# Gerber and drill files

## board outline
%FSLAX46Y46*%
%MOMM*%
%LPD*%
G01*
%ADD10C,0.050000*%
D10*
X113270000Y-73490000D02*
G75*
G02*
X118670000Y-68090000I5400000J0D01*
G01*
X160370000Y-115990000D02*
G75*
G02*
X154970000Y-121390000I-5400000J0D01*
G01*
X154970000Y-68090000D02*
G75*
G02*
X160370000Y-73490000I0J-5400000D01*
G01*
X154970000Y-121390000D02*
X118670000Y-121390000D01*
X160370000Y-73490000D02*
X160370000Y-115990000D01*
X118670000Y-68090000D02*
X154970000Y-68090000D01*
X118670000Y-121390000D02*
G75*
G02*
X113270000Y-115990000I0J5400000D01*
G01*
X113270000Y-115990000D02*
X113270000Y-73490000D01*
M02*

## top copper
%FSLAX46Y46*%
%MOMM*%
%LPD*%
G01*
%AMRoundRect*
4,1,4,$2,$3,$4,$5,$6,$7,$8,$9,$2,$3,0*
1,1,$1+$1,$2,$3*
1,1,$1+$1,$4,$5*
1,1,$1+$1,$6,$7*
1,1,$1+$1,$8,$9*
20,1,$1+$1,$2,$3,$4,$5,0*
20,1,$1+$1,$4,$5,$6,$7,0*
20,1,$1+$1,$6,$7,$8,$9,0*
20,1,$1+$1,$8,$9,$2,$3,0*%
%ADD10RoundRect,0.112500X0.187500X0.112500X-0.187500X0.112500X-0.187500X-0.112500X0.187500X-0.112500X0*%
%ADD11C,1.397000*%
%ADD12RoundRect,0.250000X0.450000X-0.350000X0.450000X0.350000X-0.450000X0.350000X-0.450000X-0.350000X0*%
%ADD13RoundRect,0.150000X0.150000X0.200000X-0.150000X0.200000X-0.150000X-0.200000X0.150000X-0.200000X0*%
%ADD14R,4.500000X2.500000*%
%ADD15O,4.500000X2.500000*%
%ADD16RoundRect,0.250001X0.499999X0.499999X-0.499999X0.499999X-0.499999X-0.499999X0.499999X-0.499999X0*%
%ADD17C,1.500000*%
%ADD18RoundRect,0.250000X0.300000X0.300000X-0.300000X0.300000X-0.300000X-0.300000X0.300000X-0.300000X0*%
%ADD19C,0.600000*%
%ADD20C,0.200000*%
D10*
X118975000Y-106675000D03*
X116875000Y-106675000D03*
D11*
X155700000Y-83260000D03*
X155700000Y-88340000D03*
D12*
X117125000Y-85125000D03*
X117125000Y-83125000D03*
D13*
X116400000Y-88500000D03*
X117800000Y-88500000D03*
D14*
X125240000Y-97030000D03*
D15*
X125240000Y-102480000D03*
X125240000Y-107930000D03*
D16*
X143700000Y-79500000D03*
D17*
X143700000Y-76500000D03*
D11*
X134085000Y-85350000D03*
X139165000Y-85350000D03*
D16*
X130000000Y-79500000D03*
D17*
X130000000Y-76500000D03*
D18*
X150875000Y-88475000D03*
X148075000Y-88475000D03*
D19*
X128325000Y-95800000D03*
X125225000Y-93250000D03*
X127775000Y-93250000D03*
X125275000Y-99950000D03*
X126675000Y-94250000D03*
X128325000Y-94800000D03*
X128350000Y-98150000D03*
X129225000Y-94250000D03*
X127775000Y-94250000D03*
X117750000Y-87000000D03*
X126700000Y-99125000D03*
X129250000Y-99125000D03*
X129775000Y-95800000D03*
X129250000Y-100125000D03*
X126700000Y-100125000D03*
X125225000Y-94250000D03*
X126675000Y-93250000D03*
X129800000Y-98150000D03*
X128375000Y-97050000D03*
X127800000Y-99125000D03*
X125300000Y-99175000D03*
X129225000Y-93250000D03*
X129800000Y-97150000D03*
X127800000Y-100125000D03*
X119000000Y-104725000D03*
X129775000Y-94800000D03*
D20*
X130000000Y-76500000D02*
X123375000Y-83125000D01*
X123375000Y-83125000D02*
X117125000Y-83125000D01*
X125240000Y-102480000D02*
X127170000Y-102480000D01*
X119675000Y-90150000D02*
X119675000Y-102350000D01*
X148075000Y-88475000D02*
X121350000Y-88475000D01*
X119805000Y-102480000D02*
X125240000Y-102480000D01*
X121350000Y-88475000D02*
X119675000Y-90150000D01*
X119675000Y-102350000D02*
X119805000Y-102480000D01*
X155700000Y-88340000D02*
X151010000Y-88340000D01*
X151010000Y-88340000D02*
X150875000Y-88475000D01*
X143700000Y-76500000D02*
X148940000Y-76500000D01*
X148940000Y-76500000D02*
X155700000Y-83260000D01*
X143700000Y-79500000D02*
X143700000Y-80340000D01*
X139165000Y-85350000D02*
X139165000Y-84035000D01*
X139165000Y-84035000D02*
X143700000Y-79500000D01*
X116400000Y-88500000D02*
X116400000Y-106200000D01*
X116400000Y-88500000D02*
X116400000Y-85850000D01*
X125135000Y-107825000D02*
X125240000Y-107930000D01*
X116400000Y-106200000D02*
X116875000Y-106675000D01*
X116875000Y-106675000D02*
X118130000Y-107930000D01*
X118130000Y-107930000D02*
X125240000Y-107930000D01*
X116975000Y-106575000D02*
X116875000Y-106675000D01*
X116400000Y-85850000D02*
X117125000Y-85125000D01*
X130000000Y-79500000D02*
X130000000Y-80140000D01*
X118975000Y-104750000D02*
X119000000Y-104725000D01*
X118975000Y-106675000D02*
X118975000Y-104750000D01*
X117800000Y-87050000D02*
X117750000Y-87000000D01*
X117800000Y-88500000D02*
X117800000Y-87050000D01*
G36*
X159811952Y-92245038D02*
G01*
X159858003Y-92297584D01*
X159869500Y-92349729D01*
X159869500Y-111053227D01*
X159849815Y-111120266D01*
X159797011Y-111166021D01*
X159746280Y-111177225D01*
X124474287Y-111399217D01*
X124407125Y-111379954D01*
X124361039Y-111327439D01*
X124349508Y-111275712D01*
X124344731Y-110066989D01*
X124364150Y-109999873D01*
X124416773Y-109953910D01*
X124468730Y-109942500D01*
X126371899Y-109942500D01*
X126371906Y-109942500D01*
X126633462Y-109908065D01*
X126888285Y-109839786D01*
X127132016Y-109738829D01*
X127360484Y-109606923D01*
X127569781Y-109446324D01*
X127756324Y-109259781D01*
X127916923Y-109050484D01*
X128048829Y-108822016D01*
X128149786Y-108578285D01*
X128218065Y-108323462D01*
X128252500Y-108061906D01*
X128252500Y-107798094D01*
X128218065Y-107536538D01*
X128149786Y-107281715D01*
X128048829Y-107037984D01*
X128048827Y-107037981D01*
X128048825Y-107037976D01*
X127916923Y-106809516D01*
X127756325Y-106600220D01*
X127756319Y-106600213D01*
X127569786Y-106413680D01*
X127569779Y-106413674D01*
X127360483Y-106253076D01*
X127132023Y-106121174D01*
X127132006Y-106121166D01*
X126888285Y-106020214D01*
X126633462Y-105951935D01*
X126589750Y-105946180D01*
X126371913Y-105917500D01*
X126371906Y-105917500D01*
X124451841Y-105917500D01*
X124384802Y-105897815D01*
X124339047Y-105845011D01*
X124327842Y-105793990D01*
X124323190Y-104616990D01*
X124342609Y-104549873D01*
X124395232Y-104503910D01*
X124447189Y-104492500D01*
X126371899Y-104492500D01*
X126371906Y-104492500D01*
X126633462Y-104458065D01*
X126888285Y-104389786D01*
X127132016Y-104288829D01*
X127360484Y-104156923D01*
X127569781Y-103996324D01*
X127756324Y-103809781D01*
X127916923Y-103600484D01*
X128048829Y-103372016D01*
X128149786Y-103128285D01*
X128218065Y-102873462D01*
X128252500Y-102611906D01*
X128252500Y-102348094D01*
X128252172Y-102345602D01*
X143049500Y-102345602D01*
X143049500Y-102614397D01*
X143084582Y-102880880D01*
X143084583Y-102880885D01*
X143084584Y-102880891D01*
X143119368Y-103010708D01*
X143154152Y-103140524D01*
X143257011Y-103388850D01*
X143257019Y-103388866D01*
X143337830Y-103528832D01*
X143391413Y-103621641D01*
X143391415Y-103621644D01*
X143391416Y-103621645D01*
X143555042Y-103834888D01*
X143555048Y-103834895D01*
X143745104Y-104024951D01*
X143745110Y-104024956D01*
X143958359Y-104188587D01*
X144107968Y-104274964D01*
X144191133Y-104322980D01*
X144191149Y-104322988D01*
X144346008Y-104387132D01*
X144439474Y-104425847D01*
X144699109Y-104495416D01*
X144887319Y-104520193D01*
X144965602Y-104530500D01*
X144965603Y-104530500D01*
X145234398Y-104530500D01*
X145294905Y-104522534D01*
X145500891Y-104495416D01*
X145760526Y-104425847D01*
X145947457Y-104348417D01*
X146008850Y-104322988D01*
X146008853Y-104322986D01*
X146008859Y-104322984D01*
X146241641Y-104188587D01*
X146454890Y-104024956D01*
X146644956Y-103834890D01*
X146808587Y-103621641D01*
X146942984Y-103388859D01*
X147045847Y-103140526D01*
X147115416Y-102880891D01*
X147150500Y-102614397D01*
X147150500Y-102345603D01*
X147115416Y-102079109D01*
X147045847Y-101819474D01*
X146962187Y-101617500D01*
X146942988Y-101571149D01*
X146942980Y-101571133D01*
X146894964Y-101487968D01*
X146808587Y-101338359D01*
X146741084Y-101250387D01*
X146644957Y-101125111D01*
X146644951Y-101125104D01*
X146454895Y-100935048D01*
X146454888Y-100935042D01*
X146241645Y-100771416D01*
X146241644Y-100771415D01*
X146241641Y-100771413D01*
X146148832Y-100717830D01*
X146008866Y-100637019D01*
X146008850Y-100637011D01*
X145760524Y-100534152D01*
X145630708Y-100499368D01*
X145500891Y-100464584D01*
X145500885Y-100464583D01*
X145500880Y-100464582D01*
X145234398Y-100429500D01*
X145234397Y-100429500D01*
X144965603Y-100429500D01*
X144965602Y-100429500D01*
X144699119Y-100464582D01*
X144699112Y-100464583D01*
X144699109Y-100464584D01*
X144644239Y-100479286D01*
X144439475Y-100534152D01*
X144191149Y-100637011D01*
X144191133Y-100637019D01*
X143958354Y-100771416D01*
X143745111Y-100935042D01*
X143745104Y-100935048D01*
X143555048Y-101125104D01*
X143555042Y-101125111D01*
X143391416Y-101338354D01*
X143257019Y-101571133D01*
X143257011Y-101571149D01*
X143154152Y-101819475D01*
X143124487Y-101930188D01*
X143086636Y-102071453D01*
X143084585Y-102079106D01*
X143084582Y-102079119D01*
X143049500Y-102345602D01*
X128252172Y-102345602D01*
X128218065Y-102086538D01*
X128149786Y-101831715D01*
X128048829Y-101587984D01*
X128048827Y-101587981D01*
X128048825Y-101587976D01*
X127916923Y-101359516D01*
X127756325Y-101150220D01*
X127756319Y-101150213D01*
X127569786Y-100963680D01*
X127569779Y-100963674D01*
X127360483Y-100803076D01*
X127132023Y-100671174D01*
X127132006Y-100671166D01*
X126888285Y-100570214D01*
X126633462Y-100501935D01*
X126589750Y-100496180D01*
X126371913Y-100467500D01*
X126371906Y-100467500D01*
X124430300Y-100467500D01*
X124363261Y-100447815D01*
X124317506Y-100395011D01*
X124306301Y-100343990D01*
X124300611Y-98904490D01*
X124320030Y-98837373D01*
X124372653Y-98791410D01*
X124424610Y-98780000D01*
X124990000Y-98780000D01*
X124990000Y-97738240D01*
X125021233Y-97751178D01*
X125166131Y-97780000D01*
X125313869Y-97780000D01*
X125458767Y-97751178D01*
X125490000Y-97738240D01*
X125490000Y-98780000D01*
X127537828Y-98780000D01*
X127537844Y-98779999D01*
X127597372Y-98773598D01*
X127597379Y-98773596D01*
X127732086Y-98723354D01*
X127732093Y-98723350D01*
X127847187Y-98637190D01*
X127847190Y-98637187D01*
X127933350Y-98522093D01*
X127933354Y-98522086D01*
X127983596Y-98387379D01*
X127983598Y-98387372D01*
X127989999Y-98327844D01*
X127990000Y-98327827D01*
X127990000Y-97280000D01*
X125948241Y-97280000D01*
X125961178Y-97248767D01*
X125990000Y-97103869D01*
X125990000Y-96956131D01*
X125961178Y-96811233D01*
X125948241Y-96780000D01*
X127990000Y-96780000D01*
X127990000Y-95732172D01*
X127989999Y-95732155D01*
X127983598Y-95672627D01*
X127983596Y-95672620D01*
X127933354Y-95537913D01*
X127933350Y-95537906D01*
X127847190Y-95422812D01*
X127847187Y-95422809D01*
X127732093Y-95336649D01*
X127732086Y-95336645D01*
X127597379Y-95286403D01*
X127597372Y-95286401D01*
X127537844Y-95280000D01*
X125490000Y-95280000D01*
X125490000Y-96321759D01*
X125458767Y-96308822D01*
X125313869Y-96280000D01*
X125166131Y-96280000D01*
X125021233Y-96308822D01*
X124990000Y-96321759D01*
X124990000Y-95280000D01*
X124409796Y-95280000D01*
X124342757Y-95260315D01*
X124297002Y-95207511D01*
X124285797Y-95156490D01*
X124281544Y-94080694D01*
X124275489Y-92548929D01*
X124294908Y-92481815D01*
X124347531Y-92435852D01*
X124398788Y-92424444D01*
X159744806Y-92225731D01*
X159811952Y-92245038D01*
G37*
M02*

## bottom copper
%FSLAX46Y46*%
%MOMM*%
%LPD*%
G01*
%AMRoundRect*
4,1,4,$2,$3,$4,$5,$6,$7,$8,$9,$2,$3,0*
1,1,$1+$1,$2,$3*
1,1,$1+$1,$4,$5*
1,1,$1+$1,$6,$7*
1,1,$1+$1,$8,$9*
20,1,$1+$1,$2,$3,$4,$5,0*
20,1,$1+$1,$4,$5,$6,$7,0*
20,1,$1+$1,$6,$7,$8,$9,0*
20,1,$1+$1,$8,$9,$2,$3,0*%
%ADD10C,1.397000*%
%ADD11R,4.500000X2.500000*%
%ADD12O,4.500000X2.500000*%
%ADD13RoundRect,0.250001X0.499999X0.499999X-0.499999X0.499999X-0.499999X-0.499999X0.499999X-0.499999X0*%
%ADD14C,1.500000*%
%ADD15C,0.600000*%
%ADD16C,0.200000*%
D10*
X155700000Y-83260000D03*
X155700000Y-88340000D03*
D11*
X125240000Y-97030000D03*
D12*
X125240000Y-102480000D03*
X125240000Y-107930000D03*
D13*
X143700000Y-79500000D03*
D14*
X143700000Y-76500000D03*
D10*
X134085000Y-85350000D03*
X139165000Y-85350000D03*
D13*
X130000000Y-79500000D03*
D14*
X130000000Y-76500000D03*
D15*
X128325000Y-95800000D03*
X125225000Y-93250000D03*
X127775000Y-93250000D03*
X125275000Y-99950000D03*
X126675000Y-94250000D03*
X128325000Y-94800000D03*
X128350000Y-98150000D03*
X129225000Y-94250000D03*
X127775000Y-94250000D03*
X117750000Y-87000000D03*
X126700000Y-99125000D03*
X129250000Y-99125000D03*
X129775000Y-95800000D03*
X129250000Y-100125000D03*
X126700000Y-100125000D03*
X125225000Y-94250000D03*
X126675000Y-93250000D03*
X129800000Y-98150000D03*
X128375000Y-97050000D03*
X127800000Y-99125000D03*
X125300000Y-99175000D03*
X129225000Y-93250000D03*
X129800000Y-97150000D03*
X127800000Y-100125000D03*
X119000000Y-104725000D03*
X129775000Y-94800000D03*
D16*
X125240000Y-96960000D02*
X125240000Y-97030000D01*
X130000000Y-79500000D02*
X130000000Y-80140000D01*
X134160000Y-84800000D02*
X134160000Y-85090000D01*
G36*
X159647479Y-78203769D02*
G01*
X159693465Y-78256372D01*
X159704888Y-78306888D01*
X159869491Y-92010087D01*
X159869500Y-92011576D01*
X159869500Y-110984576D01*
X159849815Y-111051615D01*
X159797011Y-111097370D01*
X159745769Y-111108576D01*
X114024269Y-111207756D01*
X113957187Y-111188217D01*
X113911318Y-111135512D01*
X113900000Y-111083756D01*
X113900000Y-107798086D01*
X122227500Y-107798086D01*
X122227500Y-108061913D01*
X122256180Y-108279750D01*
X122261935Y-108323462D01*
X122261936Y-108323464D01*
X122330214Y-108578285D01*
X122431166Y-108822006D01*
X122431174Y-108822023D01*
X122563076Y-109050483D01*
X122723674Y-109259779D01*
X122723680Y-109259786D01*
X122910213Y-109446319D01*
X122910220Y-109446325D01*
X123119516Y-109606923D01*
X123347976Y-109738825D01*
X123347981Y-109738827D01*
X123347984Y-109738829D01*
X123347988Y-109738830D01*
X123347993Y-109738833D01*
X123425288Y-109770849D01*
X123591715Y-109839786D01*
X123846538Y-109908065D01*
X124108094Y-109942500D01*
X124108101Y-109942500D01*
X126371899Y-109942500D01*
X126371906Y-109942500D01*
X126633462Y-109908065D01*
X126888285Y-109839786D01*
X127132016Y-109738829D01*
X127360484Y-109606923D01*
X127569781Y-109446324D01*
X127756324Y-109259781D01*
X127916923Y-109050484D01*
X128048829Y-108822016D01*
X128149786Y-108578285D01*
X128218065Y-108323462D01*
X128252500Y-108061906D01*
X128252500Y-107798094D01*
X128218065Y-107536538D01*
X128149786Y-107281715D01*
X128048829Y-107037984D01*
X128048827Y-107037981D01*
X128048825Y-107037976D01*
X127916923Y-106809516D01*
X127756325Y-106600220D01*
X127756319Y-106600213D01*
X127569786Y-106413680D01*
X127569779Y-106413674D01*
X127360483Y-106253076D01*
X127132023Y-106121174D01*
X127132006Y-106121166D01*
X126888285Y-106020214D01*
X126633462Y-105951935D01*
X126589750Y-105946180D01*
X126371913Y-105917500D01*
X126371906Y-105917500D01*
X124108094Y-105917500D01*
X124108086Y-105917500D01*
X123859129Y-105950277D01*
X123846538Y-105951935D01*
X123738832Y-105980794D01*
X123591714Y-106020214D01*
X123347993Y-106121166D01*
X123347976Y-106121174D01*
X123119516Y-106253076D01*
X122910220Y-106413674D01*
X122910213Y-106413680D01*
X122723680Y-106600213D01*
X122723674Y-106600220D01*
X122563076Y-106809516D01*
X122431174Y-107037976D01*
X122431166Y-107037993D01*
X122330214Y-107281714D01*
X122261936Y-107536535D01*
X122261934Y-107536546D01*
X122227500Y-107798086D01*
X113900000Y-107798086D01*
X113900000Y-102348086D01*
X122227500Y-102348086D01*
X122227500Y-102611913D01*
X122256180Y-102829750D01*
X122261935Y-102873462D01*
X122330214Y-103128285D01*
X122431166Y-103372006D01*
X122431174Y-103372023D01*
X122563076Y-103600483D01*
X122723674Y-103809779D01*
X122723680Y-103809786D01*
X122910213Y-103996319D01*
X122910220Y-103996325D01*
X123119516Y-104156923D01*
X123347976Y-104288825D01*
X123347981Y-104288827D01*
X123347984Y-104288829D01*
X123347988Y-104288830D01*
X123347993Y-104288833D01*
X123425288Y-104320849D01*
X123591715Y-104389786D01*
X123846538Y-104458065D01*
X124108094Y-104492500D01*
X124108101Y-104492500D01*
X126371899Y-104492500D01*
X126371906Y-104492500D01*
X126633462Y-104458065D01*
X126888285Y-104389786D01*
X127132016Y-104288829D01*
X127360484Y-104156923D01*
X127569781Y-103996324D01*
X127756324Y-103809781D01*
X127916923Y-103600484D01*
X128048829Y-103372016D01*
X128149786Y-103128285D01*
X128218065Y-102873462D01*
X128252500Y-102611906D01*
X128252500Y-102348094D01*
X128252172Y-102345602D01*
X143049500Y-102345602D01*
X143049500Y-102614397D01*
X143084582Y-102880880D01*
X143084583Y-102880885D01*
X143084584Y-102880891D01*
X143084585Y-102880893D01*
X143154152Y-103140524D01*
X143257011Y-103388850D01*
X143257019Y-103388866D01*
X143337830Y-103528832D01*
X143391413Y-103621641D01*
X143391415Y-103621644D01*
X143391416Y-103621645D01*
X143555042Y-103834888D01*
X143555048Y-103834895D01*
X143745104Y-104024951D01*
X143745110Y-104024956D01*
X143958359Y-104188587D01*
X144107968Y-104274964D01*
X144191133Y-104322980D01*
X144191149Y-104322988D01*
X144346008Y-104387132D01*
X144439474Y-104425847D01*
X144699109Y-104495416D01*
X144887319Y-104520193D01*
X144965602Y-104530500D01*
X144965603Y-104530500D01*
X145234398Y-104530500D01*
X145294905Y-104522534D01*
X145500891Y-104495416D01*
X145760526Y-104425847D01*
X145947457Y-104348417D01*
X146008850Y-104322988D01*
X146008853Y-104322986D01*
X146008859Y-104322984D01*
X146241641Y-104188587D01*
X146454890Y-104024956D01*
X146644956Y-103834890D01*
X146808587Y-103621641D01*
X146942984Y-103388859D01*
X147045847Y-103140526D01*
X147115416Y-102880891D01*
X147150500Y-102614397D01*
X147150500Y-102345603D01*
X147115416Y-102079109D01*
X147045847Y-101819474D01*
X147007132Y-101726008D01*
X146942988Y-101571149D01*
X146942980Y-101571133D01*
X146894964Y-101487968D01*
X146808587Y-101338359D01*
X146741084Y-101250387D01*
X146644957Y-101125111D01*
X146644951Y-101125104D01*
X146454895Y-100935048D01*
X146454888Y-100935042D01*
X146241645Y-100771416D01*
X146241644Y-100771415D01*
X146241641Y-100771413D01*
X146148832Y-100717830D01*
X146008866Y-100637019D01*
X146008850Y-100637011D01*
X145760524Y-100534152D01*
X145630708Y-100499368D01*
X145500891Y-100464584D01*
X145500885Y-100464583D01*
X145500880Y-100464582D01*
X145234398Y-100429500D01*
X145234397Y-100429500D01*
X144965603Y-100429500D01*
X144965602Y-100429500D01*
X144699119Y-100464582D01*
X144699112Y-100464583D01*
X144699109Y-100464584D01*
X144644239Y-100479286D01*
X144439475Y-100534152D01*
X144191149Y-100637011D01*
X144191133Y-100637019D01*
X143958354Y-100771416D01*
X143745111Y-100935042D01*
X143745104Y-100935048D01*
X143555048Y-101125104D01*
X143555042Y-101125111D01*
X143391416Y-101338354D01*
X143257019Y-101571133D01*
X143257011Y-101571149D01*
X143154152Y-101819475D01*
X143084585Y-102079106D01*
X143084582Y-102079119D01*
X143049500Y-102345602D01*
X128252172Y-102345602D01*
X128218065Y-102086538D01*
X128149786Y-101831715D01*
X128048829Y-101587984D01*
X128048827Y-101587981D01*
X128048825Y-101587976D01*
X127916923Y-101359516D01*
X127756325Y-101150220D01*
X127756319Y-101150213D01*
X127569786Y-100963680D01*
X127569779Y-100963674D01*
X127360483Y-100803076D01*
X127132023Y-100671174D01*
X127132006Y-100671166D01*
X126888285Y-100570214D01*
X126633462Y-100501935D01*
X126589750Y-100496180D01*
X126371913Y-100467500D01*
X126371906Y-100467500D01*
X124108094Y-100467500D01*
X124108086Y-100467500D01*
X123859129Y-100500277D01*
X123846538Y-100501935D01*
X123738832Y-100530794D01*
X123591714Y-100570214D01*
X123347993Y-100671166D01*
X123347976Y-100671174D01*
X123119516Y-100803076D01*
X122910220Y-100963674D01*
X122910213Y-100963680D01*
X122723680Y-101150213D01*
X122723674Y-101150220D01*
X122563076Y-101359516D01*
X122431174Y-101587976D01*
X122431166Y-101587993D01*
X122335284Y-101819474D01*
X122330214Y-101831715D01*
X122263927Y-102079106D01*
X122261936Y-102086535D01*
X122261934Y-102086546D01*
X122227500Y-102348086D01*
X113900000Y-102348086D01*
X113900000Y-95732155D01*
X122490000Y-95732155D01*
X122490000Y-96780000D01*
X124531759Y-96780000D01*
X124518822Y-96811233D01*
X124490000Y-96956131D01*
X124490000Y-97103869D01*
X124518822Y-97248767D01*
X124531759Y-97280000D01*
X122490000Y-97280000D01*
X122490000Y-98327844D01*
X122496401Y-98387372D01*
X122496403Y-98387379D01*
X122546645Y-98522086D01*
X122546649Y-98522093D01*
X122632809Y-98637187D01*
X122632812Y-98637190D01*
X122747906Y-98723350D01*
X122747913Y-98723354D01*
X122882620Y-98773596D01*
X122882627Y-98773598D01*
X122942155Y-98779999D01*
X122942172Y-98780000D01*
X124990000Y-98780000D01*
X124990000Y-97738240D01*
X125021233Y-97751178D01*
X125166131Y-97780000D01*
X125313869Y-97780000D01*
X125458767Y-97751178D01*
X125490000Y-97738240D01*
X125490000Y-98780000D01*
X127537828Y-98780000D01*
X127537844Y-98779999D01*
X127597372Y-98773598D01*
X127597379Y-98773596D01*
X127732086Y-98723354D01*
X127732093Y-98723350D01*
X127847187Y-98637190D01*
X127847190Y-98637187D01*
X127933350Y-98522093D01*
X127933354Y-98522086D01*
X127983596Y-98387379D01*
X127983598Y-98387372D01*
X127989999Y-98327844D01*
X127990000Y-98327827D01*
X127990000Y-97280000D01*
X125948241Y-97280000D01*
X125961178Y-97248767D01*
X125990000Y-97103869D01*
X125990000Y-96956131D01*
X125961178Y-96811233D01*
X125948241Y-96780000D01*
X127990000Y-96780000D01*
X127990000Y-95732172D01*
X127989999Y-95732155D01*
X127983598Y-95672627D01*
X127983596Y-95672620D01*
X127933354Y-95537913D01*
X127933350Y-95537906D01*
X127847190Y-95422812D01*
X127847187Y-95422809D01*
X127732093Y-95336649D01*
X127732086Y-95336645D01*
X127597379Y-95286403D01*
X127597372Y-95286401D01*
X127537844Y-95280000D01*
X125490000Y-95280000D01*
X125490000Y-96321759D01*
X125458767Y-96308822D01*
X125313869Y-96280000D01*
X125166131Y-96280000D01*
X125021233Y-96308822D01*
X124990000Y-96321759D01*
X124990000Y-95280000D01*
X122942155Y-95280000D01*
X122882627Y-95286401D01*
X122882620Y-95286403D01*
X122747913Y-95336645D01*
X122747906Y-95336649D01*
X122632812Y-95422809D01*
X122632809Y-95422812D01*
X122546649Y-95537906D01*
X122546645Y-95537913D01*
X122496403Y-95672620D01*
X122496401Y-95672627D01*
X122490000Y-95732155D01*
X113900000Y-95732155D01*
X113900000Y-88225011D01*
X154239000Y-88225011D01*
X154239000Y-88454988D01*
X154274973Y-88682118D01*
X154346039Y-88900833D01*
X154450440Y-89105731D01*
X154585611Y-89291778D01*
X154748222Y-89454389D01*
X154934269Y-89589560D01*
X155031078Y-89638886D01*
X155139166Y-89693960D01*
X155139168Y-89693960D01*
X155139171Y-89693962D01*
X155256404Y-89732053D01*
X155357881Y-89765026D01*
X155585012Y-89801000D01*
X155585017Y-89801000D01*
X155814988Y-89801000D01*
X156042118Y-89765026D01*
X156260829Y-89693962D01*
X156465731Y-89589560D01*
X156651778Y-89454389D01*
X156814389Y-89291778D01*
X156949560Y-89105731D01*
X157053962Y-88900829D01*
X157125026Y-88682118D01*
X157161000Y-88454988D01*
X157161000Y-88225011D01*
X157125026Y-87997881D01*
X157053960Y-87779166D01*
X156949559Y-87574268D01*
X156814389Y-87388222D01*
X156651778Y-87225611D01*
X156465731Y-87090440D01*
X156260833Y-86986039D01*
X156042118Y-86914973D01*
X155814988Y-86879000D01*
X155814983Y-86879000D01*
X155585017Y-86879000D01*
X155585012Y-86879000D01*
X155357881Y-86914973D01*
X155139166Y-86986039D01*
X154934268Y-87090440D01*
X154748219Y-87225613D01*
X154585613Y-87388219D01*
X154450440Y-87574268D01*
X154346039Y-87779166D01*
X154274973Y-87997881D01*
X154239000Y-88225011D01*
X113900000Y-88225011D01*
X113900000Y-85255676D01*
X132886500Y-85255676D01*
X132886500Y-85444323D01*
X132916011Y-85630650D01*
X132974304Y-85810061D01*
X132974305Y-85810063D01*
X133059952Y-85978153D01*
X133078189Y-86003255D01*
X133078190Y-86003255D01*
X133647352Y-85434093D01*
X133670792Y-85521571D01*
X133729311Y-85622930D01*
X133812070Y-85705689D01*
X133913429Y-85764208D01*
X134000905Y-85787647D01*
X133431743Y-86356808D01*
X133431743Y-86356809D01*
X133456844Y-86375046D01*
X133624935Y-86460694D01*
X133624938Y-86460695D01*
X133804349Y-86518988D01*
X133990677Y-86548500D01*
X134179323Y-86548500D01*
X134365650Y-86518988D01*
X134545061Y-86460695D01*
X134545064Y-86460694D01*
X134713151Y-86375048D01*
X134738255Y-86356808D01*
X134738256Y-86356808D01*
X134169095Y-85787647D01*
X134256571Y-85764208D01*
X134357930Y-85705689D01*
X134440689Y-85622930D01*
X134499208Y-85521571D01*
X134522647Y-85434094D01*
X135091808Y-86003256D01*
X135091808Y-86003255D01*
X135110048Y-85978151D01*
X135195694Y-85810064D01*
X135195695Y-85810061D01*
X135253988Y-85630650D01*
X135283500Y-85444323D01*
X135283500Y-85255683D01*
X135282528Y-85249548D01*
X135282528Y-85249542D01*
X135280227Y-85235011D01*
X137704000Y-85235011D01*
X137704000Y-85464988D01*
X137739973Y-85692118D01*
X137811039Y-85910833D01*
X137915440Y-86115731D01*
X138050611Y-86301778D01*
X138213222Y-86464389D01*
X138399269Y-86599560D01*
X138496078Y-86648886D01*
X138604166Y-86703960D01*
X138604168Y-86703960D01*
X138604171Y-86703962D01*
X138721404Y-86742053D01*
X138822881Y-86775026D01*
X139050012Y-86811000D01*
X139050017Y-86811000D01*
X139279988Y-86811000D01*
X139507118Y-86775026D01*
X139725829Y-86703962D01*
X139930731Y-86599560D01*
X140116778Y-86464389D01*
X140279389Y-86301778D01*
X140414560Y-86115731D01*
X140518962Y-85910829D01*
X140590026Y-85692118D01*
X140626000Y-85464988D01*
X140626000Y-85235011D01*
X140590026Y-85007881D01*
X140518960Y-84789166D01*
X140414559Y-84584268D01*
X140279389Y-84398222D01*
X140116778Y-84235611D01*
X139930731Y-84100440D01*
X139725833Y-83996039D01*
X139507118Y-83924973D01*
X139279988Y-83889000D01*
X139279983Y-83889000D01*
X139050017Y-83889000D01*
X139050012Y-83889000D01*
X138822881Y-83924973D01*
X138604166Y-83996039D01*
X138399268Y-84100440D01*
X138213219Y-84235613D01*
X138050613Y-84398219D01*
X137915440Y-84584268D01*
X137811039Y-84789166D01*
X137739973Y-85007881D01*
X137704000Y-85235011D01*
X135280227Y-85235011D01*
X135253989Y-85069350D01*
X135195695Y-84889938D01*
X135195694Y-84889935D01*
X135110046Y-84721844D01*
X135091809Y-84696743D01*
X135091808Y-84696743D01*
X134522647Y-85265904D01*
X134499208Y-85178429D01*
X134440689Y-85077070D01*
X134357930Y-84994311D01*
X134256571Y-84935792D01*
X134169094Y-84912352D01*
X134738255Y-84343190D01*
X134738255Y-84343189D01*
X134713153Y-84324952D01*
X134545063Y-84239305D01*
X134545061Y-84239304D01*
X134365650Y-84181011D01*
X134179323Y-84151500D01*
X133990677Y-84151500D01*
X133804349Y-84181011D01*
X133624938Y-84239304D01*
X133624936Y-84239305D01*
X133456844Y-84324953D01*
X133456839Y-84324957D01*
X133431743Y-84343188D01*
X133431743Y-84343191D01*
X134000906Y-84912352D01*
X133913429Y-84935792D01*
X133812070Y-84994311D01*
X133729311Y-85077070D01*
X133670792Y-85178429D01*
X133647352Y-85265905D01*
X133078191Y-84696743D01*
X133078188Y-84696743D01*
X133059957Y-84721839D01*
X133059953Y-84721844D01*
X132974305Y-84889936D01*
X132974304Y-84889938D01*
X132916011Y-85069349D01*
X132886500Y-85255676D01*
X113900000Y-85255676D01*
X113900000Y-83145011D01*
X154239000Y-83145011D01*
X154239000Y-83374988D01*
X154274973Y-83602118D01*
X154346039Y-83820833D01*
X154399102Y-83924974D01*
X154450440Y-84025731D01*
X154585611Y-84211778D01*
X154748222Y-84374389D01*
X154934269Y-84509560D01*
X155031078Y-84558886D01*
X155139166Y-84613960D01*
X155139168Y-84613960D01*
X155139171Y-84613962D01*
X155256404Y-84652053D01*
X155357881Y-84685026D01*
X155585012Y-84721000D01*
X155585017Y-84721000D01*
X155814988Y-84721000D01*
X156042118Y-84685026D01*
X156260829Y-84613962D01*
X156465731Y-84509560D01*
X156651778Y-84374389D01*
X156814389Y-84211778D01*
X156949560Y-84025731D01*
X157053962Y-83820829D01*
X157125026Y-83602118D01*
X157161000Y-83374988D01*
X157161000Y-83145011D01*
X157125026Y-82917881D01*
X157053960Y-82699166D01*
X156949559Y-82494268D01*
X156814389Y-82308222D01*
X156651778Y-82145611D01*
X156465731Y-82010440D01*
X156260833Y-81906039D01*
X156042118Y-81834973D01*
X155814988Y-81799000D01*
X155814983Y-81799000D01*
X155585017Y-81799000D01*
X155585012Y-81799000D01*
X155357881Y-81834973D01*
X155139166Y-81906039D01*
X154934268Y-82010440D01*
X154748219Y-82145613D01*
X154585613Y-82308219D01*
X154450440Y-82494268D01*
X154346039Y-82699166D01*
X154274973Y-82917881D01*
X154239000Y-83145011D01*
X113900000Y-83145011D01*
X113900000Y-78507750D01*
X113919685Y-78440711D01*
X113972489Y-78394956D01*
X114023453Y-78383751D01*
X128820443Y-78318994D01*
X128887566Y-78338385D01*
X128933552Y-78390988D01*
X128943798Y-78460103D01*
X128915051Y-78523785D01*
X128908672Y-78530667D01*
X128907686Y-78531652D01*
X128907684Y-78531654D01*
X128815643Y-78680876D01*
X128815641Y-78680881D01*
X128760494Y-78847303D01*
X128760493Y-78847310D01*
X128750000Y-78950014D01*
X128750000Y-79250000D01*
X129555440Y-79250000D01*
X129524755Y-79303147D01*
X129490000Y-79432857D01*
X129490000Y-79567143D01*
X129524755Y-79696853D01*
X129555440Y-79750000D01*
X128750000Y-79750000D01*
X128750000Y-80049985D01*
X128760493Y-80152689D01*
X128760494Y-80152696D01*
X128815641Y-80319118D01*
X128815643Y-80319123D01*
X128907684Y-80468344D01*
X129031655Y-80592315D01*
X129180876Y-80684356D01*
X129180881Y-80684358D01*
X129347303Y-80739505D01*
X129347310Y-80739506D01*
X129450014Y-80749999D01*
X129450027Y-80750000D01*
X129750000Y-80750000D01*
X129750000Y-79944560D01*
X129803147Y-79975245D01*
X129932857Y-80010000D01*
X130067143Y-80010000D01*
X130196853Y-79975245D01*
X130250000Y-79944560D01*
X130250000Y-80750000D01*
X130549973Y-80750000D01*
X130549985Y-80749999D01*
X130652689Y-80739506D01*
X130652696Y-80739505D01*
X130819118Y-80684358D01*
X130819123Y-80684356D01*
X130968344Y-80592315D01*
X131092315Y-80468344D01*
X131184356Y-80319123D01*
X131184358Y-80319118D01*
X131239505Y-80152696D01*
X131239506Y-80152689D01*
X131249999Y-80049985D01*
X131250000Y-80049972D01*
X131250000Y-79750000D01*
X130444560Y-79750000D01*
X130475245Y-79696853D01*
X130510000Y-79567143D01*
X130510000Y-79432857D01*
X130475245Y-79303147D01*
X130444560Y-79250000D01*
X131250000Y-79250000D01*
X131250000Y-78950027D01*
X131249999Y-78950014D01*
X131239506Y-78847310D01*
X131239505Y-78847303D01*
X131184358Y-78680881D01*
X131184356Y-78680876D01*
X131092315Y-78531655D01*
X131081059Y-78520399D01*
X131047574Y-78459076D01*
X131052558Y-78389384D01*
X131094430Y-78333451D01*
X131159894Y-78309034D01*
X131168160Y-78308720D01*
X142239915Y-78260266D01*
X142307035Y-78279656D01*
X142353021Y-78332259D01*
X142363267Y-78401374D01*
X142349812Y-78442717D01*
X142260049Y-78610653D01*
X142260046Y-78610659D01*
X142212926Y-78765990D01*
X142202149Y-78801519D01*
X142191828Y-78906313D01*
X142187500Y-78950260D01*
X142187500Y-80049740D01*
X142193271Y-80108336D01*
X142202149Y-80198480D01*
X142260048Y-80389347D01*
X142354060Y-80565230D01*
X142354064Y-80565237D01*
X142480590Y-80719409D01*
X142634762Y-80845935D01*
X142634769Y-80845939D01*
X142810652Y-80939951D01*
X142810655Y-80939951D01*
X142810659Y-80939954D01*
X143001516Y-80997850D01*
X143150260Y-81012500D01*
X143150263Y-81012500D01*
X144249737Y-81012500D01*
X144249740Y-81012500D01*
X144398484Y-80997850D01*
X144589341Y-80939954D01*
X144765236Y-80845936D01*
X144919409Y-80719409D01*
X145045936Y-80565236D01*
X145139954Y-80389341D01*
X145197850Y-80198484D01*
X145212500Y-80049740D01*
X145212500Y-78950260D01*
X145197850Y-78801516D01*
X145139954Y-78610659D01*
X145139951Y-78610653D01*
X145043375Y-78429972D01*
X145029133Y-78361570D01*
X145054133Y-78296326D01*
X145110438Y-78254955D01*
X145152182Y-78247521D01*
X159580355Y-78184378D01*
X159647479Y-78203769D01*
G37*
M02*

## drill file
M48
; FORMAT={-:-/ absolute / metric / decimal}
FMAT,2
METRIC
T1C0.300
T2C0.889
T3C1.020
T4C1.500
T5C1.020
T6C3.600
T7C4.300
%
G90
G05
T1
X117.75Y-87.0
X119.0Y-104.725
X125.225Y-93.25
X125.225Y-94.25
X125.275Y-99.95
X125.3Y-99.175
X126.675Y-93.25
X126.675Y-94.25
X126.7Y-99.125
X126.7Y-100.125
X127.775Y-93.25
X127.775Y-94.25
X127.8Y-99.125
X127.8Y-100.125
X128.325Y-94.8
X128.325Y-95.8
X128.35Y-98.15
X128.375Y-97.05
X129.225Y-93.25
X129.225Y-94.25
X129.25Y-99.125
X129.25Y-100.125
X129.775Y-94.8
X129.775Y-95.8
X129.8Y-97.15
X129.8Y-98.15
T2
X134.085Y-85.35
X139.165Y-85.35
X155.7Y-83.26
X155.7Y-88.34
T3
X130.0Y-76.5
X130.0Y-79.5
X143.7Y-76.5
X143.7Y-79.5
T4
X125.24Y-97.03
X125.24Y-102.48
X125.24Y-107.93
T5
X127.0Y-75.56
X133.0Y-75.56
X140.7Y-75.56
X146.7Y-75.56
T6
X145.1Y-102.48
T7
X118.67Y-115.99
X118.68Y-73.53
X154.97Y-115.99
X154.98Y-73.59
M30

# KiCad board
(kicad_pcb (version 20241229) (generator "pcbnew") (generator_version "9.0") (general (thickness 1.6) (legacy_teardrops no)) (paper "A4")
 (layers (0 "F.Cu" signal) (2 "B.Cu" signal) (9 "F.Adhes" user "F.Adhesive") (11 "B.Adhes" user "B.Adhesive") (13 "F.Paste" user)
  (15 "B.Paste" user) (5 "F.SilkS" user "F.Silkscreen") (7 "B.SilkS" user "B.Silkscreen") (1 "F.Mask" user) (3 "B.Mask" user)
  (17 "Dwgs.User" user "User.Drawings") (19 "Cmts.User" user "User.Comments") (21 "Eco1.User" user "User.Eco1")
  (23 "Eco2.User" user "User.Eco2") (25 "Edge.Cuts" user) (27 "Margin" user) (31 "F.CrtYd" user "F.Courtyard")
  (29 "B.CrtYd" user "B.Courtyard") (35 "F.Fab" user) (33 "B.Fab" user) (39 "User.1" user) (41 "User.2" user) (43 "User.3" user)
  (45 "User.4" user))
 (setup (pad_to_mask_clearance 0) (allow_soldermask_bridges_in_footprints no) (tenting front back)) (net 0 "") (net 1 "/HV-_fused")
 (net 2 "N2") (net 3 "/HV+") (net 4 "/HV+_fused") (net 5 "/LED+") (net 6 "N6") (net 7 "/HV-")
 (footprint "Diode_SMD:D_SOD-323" (layer "F.Cu") (at 117.925 106.675 180)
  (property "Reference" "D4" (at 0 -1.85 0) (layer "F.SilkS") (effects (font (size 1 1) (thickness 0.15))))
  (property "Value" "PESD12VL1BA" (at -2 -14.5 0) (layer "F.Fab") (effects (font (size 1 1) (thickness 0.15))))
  (pad "1" smd roundrect (at -1.05 0 180) (size 0.6 0.45) (layers "F.Cu" "F.Mask" "F.Paste") (roundrect_rratio 0.25) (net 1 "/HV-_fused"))
  (pad "2" smd roundrect (at 1.05 0 180) (size 0.6 0.45) (layers "F.Cu" "F.Mask" "F.Paste") (roundrect_rratio 0.25) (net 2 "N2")))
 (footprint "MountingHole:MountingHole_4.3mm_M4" (layer "F.Cu") (at 118.679999 73.53 180)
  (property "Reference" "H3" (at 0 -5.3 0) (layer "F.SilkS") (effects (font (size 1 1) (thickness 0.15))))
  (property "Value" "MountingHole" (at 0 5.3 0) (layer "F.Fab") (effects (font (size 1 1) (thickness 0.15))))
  (pad "" np_thru_hole circle (at 0 0 180) (size 4.3 4.3) (drill 4.3) (layers "*.Cu" "*.Mask")))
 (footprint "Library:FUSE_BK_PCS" (layer "F.Cu") (at 155.7 85.8 -90)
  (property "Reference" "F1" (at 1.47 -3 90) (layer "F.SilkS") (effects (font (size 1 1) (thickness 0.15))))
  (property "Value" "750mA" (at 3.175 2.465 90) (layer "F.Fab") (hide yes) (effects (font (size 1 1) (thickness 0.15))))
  (pad "1" thru_hole circle (at -2.54 0 270) (size 1.397 1.397) (drill 0.889) (layers "*.Cu" "*.Mask") (remove_unused_layers no)
   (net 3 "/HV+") (solder_mask_margin 0.102))
  (pad "2" thru_hole circle (at 2.54 0 270) (size 1.397 1.397) (drill 0.889) (layers "*.Cu" "*.Mask") (remove_unused_layers no)
   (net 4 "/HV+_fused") (solder_mask_margin 0.102)))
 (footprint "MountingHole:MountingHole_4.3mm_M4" (layer "F.Cu") (at 118.669999 115.990001)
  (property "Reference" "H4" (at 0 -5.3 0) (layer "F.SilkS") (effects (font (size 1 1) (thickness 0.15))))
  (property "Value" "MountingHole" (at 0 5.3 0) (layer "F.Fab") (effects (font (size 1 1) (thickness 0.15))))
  (pad "" np_thru_hole circle (at 0 0) (size 4.3 4.3) (drill 4.3) (layers "*.Cu" "*.Mask")))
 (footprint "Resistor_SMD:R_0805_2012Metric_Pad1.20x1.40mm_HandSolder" (layer "F.Cu") (at 117.125 84.125 90)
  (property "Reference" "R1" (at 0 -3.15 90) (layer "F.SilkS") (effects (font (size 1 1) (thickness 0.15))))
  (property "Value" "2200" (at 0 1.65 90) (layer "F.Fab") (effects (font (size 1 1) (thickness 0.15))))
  (pad "1" smd roundrect (at -1 0 90) (size 1.2 1.4) (layers "F.Cu" "F.Mask" "F.Paste") (roundrect_rratio 0.208333) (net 2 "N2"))
  (pad "2" smd roundrect (at 1 0 90) (size 1.2 1.4) (layers "F.Cu" "F.Mask" "F.Paste") (roundrect_rratio 0.208333) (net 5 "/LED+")))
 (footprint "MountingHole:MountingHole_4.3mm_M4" (layer "F.Cu") (at 154.980001 73.59 180)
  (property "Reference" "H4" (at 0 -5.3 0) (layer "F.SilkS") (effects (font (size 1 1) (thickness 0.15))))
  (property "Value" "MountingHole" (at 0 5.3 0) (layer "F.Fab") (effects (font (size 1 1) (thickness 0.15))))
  (pad "" np_thru_hole circle (at 0 0 180) (size 4.3 4.3) (drill 4.3) (layers "*.Cu" "*.Mask")))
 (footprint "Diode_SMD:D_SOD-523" (layer "F.Cu") (at 117.1 88.5)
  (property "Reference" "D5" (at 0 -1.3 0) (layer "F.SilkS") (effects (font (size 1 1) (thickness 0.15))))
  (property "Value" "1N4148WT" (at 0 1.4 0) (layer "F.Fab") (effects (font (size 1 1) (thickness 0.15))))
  (pad "1" smd roundrect (at -0.7 0 180) (size 0.6 0.7) (layers "F.Cu" "F.Mask" "F.Paste") (roundrect_rratio 0.25) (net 2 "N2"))
  (pad "2" smd roundrect (at 0.7 0 180) (size 0.6 0.7) (layers "F.Cu" "F.Mask" "F.Paste") (roundrect_rratio 0.25) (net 1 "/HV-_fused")))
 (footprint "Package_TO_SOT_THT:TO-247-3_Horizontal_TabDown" (layer "F.Cu") (at 125.24 97.03 -90)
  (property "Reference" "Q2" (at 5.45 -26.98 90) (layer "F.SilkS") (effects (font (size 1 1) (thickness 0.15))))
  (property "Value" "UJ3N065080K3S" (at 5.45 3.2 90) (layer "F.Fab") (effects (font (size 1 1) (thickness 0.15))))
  (pad "" np_thru_hole circle (at 5.45 -19.86 270) (size 3.6 3.6) (drill 3.6) (layers "*.Cu" "*.Mask"))
  (pad "1" thru_hole rect (at 0 0 270) (size 2.5 4.5) (drill 1.5) (layers "*.Cu" "*.Mask") (remove_unused_layers no) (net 1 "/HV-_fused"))
  (pad "2" thru_hole oval (at 5.45 0 270) (size 2.5 4.5) (drill 1.5) (layers "*.Cu" "*.Mask") (remove_unused_layers no) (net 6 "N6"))
  (pad "3" thru_hole oval (at 10.9 0 270) (size 2.5 4.5) (drill 1.5) (layers "*.Cu" "*.Mask") (remove_unused_layers no) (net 2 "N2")))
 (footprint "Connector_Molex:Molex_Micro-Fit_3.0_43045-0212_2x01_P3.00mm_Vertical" (layer "F.Cu") (at 143.7 79.5 180)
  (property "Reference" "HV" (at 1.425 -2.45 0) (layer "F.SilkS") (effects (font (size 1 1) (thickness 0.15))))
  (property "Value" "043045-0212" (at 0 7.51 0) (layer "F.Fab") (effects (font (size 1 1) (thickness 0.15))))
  (pad "" np_thru_hole circle (at -3 3.94 180) (size 1.02 1.02) (drill 1.02) (layers "*.Cu" "*.Mask"))
  (pad "" np_thru_hole circle (at 3 3.94 180) (size 1.02 1.02) (drill 1.02) (layers "*.Cu" "*.Mask"))
  (pad "1" thru_hole roundrect (at 0 0 180) (size 1.5 1.5) (drill 1.02) (layers "*.Cu" "*.Mask") (remove_unused_layers no)
   (roundrect_rratio 0.166667) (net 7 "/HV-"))
  (pad "2" thru_hole circle (at 0 3 180) (size 1.5 1.5) (drill 1.02) (layers "*.Cu" "*.Mask") (remove_unused_layers no) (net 3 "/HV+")))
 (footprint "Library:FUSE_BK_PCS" (layer "F.Cu") (at 136.625 85.35)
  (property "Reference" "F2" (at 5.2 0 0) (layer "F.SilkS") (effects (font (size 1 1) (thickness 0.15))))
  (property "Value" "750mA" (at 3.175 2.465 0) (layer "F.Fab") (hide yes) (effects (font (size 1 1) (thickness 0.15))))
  (pad "1" thru_hole circle (at -2.54 0) (size 1.397 1.397) (drill 0.889) (layers "*.Cu" "*.Mask") (remove_unused_layers no)
   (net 1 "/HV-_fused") (solder_mask_margin 0.102))
  (pad "2" thru_hole circle (at 2.54 0) (size 1.397 1.397) (drill 0.889) (layers "*.Cu" "*.Mask") (remove_unused_layers no) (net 7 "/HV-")
   (solder_mask_margin 0.102)))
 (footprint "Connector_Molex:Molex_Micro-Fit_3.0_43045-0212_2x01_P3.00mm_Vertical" (layer "F.Cu") (at 130 79.5 180)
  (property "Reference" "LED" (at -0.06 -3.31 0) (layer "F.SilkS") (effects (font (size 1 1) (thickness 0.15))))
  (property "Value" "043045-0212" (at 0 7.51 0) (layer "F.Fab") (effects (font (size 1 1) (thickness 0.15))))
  (pad "" np_thru_hole circle (at -3 3.94 180) (size 1.02 1.02) (drill 1.02) (layers "*.Cu" "*.Mask"))
  (pad "" np_thru_hole circle (at 3 3.94 180) (size 1.02 1.02) (drill 1.02) (layers "*.Cu" "*.Mask"))
  (pad "1" thru_hole roundrect (at 0 0 180) (size 1.5 1.5) (drill 1.02) (layers "*.Cu" "*.Mask") (remove_unused_layers no)
   (roundrect_rratio 0.166667) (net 1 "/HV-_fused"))
  (pad "2" thru_hole circle (at 0 3 180) (size 1.5 1.5) (drill 1.02) (layers "*.Cu" "*.Mask") (remove_unused_layers no) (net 5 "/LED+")))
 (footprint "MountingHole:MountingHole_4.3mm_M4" (layer "F.Cu") (at 154.970001 115.990001)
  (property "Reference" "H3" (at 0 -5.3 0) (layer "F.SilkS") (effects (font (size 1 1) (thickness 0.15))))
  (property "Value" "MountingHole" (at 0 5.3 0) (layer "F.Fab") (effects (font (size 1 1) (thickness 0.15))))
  (pad "" np_thru_hole circle (at 0 0) (size 4.3 4.3) (drill 4.3) (layers "*.Cu" "*.Mask")))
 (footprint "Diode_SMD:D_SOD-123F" (layer "F.Cu") (at 149.475 88.475 180)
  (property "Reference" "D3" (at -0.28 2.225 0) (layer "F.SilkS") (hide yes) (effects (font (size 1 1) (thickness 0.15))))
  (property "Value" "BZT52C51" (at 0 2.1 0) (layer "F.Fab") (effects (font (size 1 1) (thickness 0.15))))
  (pad "1" smd roundrect (at -1.4 0 180) (size 1.1 1.1) (layers "F.Cu" "F.Mask" "F.Paste") (roundrect_rratio 0.2272727273)
   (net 4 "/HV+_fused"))
  (pad "2" smd roundrect (at 1.4 0 180) (size 1.1 1.1) (layers "F.Cu" "F.Mask" "F.Paste") (roundrect_rratio 0.2272727273) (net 6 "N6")))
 (gr_arc (start 113.27 73.49) (mid 114.851623 69.671623) (end 118.67 68.09) (stroke (width 0.05) (type default)) (layer "Edge.Cuts"))
 (gr_arc (start 160.37 115.99) (mid 158.788377 119.808377) (end 154.97 121.39) (stroke (width 0.05) (type default)) (layer "Edge.Cuts"))
 (gr_arc (start 154.97 68.09) (mid 158.788377 69.671623) (end 160.37 73.49) (stroke (width 0.05) (type default)) (layer "Edge.Cuts"))
 (gr_line (start 154.97 121.39) (end 118.67 121.39) (stroke (width 0.05) (type default)) (layer "Edge.Cuts"))
 (gr_line (start 160.37 73.49) (end 160.37 115.99) (stroke (width 0.05) (type default)) (layer "Edge.Cuts"))
 (gr_line (start 118.67 68.09) (end 154.97 68.09) (stroke (width 0.05) (type default)) (layer "Edge.Cuts"))
 (gr_arc (start 118.67 121.39) (mid 114.851623 119.808377) (end 113.27 115.99) (stroke (width 0.05) (type default)) (layer "Edge.Cuts"))
 (gr_line (start 113.27 115.99) (end 113.27 73.49) (stroke (width 0.05) (type default)) (layer "Edge.Cuts"))
 (segment (start 130 76.5) (end 123.375 83.125) (width 0.2) (layer "F.Cu") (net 5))
 (segment (start 123.375 83.125) (end 117.125 83.125) (width 0.2) (layer "F.Cu") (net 5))
 (segment (start 125.24 102.48) (end 127.17 102.48) (width 0.2) (layer "F.Cu") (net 6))
 (segment (start 119.675 90.15) (end 119.675 102.35) (width 0.2) (layer "F.Cu") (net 6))
 (segment (start 148.075 88.475) (end 121.35 88.475) (width 0.2) (layer "F.Cu") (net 6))
 (segment (start 119.805 102.48) (end 125.24 102.48) (width 0.2) (layer "F.Cu") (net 6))
 (segment (start 121.35 88.475) (end 119.675 90.15) (width 0.2) (layer "F.Cu") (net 6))
 (segment (start 119.675 102.35) (end 119.805 102.48) (width 0.2) (layer "F.Cu") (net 6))
 (segment (start 155.7 88.34) (end 151.01 88.34) (width 0.2) (layer "F.Cu") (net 4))
 (segment (start 151.01 88.34) (end 150.875 88.475) (width 0.2) (layer "F.Cu") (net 4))
 (segment (start 143.7 76.5) (end 148.94 76.5) (width 0.2) (layer "F.Cu") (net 3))
 (segment (start 148.94 76.5) (end 155.7 83.26) (width 0.2) (layer "F.Cu") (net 3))
 (segment (start 143.7 79.5) (end 143.7 80.34) (width 0.2) (layer "F.Cu") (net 7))
 (segment (start 139.165 85.35) (end 139.165 84.035) (width 0.2) (layer "F.Cu") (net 7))
 (segment (start 139.165 84.035) (end 143.7 79.5) (width 0.2) (layer "F.Cu") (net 7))
 (segment (start 116.4 88.5) (end 116.4 106.2) (width 0.2) (layer "F.Cu") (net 2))
 (segment (start 116.4 88.5) (end 116.4 85.85) (width 0.2) (layer "F.Cu") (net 2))
 (segment (start 125.135 107.825) (end 125.24 107.93) (width 0.2) (layer "F.Cu") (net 2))
 (segment (start 116.4 106.2) (end 116.875 106.675) (width 0.2) (layer "F.Cu") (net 2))
 (segment (start 116.875 106.675) (end 118.13 107.93) (width 0.2) (layer "F.Cu") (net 2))
 (segment (start 118.13 107.93) (end 125.24 107.93) (width 0.2) (layer "F.Cu") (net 2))
 (segment (start 116.975 106.575) (end 116.875 106.675) (width 0.2) (layer "F.Cu") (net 2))
 (segment (start 116.4 85.85) (end 117.125 85.125) (width 0.2) (layer "F.Cu") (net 2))
 (segment (start 130 79.5) (end 130 80.14) (width 0.2) (layer "F.Cu") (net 1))
 (segment (start 118.975 104.75) (end 119 104.725) (width 0.2) (layer "F.Cu") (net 1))
 (segment (start 118.975 106.675) (end 118.975 104.75) (width 0.2) (layer "F.Cu") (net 1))
 (segment (start 117.8 87.05) (end 117.75 87) (width 0.2) (layer "F.Cu") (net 1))
 (segment (start 117.8 88.5) (end 117.8 87.05) (width 0.2) (layer "F.Cu") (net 1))
 (via (at 128.325 95.8) (size 0.6) (drill 0.3) (layers "F.Cu" "B.Cu") (free yes) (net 1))
 (via (at 125.225 93.25) (size 0.6) (drill 0.3) (layers "F.Cu" "B.Cu") (free yes) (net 1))
 (via (at 127.775 93.25) (size 0.6) (drill 0.3) (layers "F.Cu" "B.Cu") (free yes) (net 1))
 (via (at 125.275 99.95) (size 0.6) (drill 0.3) (layers "F.Cu" "B.Cu") (free yes) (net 1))
 (via (at 126.675 94.25) (size 0.6) (drill 0.3) (layers "F.Cu" "B.Cu") (free yes) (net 1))
 (via (at 128.325 94.8) (size 0.6) (drill 0.3) (layers "F.Cu" "B.Cu") (free yes) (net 1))
 (via (at 128.35 98.15) (size 0.6) (drill 0.3) (layers "F.Cu" "B.Cu") (free yes) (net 1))
 (via (at 129.225 94.25) (size 0.6) (drill 0.3) (layers "F.Cu" "B.Cu") (free yes) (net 1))
 (via (at 127.775 94.25) (size 0.6) (drill 0.3) (layers "F.Cu" "B.Cu") (free yes) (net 1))
 (via (at 117.75 87) (size 0.6) (drill 0.3) (layers "F.Cu" "B.Cu") (free yes) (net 1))
 (via (at 126.7 99.125) (size 0.6) (drill 0.3) (layers "F.Cu" "B.Cu") (free yes) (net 1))
 (via (at 129.25 99.125) (size 0.6) (drill 0.3) (layers "F.Cu" "B.Cu") (free yes) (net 1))
 (via (at 129.775 95.8) (size 0.6) (drill 0.3) (layers "F.Cu" "B.Cu") (free yes) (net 1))
 (via (at 129.25 100.125) (size 0.6) (drill 0.3) (layers "F.Cu" "B.Cu") (free yes) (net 1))
 (via (at 126.7 100.125) (size 0.6) (drill 0.3) (layers "F.Cu" "B.Cu") (free yes) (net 1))
 (via (at 125.225 94.25) (size 0.6) (drill 0.3) (layers "F.Cu" "B.Cu") (free yes) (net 1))
 (via (at 126.675 93.25) (size 0.6) (drill 0.3) (layers "F.Cu" "B.Cu") (free yes) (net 1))
 (via (at 129.8 98.15) (size 0.6) (drill 0.3) (layers "F.Cu" "B.Cu") (free yes) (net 1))
 (via (at 128.375 97.05) (size 0.6) (drill 0.3) (layers "F.Cu" "B.Cu") (free yes) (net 1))
 (via (at 127.8 99.125) (size 0.6) (drill 0.3) (layers "F.Cu" "B.Cu") (free yes) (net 1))
 (via (at 125.3 99.175) (size 0.6) (drill 0.3) (layers "F.Cu" "B.Cu") (free yes) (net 1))
 (via (at 129.225 93.25) (size 0.6) (drill 0.3) (layers "F.Cu" "B.Cu") (free yes) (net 1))
 (via (at 129.8 97.15) (size 0.6) (drill 0.3) (layers "F.Cu" "B.Cu") (free yes) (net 1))
 (via (at 127.8 100.125) (size 0.6) (drill 0.3) (layers "F.Cu" "B.Cu") (free yes) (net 1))
 (via (at 119 104.725) (size 0.6) (drill 0.3) (layers "F.Cu" "B.Cu") (free yes) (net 1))
 (via (at 129.775 94.8) (size 0.6) (drill 0.3) (layers "F.Cu" "B.Cu") (free yes) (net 1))
 (segment (start 125.24 96.96) (end 125.24 97.03) (width 0.2) (layer "B.Cu") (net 1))
 (segment (start 130 79.5) (end 130 80.14) (width 0.2) (layer "B.Cu") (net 1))
 (segment (start 134.16 84.8) (end 134.16 85.09) (width 0.2) (layer "B.Cu") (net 1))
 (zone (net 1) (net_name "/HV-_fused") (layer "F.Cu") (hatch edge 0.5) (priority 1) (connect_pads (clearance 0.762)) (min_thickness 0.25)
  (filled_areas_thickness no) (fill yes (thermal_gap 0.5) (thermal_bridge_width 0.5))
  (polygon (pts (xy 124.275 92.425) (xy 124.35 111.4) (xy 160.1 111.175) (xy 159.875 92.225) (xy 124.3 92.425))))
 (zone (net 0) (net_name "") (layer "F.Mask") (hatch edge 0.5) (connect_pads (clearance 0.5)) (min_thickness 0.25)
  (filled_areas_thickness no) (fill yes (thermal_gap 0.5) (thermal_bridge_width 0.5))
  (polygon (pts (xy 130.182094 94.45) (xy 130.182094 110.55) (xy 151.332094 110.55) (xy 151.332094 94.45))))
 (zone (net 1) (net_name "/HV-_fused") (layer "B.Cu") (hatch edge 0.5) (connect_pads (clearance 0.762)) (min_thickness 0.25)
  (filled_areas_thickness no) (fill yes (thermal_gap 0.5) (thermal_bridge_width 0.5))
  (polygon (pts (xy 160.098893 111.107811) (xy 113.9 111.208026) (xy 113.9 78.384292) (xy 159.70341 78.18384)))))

